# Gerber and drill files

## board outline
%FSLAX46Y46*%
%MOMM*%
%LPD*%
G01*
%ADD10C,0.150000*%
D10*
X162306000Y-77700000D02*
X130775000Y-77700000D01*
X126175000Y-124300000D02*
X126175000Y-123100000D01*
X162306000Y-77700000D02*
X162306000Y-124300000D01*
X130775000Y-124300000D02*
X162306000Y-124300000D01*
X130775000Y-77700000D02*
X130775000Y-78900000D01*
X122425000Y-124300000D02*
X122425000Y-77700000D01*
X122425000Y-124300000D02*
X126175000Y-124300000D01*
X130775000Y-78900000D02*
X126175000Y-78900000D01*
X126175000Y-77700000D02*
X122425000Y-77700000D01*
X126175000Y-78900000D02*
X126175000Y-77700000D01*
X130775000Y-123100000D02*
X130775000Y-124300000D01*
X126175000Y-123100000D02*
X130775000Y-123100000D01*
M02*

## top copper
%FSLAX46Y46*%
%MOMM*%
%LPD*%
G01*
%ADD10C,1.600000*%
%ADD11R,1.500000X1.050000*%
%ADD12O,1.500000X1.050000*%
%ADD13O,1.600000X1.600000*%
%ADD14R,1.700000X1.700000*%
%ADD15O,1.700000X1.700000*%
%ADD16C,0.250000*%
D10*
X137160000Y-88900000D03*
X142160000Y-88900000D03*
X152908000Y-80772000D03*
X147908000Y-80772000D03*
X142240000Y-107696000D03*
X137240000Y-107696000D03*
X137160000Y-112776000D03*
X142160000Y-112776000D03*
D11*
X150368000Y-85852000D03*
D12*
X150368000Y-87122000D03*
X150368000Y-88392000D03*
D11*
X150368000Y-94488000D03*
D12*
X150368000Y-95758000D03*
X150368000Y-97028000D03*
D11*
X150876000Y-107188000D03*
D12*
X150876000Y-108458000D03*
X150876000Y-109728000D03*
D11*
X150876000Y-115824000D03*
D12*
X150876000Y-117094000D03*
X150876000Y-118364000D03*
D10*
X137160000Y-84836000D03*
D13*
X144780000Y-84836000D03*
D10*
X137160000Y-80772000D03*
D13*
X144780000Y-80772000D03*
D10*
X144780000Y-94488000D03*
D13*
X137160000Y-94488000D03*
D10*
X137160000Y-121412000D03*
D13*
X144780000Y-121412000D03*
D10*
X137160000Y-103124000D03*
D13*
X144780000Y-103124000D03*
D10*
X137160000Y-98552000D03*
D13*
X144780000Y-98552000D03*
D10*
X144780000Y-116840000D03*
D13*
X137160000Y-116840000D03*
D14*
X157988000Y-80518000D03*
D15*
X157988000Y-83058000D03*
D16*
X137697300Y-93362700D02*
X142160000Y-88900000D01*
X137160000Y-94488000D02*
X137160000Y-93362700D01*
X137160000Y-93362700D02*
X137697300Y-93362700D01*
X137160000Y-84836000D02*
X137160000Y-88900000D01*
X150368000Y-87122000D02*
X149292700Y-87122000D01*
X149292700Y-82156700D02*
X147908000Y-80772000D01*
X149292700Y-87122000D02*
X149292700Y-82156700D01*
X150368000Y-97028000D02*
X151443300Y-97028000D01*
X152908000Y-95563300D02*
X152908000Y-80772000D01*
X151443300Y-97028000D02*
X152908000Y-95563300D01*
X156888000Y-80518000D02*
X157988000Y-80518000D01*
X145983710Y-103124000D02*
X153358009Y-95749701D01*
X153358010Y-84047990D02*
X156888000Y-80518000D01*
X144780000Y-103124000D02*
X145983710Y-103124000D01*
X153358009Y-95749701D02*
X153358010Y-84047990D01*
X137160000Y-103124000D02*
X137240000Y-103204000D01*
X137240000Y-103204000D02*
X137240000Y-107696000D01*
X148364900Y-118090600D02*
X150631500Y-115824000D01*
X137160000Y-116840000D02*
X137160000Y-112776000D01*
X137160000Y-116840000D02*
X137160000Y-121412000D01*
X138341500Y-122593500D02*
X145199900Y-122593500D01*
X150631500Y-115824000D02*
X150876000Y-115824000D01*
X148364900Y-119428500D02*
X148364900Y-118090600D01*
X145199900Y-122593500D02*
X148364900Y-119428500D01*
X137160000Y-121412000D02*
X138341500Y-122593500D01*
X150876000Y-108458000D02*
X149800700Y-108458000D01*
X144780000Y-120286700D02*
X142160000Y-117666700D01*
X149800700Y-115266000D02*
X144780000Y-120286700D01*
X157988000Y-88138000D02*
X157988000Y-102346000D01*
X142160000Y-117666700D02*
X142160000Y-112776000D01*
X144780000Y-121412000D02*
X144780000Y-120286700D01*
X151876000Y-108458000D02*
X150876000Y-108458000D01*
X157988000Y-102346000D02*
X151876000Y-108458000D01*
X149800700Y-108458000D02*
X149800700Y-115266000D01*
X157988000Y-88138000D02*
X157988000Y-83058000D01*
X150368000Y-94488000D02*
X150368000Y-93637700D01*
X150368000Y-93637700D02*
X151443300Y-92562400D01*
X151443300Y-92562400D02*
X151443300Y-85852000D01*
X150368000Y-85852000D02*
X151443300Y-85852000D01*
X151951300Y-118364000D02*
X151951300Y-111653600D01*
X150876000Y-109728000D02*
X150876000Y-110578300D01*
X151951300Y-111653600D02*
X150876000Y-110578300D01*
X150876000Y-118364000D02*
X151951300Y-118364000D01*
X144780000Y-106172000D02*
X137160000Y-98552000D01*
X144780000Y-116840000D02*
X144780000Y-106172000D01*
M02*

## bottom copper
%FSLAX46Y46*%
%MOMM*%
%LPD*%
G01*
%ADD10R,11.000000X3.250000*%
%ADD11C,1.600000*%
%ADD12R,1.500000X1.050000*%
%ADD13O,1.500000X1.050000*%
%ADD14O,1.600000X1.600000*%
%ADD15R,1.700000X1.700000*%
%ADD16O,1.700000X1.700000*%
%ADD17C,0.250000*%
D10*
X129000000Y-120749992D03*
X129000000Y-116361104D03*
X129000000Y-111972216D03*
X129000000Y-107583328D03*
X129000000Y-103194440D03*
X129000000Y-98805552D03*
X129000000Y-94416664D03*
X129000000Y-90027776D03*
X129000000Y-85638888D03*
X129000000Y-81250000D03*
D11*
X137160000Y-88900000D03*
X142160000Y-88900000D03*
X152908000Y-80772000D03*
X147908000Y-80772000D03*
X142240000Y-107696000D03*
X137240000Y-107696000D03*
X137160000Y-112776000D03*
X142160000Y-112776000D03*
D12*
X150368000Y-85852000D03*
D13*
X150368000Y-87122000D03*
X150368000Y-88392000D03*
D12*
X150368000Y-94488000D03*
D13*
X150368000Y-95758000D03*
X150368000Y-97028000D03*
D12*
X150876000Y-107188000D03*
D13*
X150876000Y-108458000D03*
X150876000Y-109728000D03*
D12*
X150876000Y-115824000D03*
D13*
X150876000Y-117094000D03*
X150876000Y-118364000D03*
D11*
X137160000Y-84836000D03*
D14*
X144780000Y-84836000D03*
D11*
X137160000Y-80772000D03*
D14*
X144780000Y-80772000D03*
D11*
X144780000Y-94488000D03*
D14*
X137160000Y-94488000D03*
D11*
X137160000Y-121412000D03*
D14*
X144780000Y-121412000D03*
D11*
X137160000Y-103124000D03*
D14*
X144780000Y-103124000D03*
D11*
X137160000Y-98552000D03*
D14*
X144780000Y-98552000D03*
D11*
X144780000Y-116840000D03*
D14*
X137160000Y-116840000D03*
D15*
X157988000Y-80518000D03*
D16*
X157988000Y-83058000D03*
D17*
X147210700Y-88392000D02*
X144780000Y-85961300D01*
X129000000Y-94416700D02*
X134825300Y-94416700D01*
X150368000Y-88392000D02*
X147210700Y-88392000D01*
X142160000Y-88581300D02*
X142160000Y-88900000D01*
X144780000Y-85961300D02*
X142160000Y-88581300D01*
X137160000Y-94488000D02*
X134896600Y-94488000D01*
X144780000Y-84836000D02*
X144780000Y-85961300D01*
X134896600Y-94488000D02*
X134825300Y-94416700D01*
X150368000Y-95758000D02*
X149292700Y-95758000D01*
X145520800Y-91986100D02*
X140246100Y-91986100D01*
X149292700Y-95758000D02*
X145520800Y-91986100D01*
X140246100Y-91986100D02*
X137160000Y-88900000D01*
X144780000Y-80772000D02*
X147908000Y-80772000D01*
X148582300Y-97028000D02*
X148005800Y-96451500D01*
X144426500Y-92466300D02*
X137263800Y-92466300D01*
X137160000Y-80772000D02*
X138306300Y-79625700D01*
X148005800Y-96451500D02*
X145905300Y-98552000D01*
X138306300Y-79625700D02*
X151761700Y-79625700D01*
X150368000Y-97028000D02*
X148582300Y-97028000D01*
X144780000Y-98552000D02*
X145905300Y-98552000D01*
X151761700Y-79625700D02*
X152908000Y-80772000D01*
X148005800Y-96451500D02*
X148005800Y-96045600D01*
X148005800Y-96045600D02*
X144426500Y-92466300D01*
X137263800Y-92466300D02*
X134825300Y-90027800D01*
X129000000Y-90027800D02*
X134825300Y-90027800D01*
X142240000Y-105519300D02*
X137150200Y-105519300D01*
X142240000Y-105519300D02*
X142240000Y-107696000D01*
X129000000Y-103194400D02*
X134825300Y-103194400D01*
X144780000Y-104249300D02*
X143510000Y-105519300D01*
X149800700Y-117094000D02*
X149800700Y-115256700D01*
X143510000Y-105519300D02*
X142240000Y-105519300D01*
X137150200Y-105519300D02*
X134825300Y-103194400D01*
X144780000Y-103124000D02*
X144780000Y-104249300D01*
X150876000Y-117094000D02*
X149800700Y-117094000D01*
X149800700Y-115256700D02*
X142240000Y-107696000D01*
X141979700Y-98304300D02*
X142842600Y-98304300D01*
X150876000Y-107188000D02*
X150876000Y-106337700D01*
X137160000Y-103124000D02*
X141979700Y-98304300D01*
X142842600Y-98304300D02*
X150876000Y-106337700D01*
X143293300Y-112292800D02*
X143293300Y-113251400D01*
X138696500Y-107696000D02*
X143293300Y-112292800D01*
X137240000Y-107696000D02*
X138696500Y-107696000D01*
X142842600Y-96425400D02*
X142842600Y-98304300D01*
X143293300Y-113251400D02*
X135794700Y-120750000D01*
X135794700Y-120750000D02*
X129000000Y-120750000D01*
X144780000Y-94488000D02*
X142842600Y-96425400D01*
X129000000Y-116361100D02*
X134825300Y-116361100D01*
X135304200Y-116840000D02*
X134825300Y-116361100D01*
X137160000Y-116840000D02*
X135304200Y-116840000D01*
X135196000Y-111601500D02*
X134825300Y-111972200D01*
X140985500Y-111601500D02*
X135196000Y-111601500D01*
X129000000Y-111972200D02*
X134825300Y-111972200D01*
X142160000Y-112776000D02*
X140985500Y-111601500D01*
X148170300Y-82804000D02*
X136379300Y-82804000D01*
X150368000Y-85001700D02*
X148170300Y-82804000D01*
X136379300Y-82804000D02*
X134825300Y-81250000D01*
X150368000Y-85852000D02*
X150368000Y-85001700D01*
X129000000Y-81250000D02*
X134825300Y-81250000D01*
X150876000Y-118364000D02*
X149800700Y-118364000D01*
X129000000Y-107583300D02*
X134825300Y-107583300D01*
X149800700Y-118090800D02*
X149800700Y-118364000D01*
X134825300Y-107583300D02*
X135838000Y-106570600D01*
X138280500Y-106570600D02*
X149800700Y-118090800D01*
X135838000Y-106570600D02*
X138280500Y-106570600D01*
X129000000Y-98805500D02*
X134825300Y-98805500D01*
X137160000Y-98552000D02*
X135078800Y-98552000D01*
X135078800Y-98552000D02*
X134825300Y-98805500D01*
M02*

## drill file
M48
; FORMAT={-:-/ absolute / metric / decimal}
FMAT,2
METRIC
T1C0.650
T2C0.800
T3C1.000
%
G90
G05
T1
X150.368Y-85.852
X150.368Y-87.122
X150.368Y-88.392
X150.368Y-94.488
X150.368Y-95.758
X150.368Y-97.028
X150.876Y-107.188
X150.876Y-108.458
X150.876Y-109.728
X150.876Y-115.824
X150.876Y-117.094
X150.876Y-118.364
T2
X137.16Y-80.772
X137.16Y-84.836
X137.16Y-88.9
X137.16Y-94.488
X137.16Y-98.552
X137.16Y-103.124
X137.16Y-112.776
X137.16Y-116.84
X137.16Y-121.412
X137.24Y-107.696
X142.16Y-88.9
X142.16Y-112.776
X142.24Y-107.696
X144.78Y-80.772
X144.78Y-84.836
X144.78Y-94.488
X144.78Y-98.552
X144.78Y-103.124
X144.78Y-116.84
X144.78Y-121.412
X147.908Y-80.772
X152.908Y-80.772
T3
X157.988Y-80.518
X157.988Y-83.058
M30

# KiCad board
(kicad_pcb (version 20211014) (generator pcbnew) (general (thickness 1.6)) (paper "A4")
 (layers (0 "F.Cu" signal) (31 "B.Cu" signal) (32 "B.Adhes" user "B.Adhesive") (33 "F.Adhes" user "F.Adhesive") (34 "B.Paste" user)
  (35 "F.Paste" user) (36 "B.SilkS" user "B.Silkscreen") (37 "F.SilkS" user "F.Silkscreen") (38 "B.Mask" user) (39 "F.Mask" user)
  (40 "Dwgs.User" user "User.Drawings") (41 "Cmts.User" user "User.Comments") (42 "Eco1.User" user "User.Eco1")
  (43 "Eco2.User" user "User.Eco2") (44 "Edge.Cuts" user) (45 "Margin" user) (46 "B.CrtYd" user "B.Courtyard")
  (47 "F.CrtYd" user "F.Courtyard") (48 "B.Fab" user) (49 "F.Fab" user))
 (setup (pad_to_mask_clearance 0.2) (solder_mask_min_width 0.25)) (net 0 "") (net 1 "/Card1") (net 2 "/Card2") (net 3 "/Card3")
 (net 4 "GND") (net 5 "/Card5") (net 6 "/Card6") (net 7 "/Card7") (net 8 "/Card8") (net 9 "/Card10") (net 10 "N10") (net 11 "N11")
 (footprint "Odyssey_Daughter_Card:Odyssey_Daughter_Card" (layer "F.Cu") (at 129 101)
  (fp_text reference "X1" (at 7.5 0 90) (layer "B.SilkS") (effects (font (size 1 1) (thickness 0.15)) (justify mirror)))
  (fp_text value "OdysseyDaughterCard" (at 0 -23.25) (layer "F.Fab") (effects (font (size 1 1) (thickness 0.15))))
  (pad "1" smd rect locked (at 0 19.749992) (size 11 3.25) (layers "B.Cu" "B.Mask") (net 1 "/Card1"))
  (pad "2" smd rect locked (at 0 15.361104) (size 11 3.25) (layers "B.Cu" "B.Mask") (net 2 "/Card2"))
  (pad "3" smd rect locked (at 0 10.972216) (size 11 3.25) (layers "B.Cu" "B.Mask") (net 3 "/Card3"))
  (pad "4" smd rect locked (at 0 6.583328) (size 11 3.25) (layers "B.Cu" "B.Mask") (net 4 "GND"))
  (pad "5" smd rect locked (at 0 2.19444) (size 11 3.25) (layers "B.Cu" "B.Mask") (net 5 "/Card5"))
  (pad "6" smd rect locked (at 0 -2.194448) (size 11 3.25) (layers "B.Cu" "B.Mask") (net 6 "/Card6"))
  (pad "7" smd rect locked (at 0 -6.583336) (size 11 3.25) (layers "B.Cu" "B.Mask") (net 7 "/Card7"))
  (pad "8" smd rect locked (at 0 -10.972224) (size 11 3.25) (layers "B.Cu" "B.Mask") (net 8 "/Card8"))
  (pad "9" smd rect locked (at 0 -15.361112) (size 11 3.25) (layers "B.Cu" "B.Mask"))
  (pad "10" smd rect locked (at 0 -19.75) (size 11 3.25) (layers "B.Cu" "B.Mask") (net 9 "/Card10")))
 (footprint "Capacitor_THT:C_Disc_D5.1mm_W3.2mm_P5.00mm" (layer "F.Cu") (at 137.16 88.9)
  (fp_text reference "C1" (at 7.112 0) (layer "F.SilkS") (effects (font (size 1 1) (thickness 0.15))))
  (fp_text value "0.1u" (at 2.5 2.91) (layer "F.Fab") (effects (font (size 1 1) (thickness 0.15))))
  (pad "1" thru_hole circle locked (at 0 0) (size 1.6 1.6) (drill 0.8) (layers *.Cu *.Mask) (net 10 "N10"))
  (pad "2" thru_hole circle locked (at 5 0) (size 1.6 1.6) (drill 0.8) (layers *.Cu *.Mask) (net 7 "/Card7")))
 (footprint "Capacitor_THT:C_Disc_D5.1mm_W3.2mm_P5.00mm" (layer "F.Cu") (at 152.908 80.772 180)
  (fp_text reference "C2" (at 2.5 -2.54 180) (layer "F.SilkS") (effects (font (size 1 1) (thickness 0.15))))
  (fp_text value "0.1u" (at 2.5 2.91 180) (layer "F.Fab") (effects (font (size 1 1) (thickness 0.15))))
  (pad "1" thru_hole circle locked (at 0 0 180) (size 1.6 1.6) (drill 0.8) (layers *.Cu *.Mask) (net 8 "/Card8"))
  (pad "2" thru_hole circle locked (at 5 0 180) (size 1.6 1.6) (drill 0.8) (layers *.Cu *.Mask) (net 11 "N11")))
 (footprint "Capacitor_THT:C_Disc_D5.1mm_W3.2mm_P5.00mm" (layer "F.Cu") (at 142.24 107.696 180)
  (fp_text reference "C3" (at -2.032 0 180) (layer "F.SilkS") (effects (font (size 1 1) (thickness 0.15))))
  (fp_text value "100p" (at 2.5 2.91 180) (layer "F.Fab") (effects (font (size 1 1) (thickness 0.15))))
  (pad "1" thru_hole circle locked (at 0 0 180) (size 1.6 1.6) (drill 0.8) (layers *.Cu *.Mask) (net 5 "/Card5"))
  (pad "2" thru_hole circle locked (at 5 0 180) (size 1.6 1.6) (drill 0.8) (layers *.Cu *.Mask) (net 1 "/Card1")))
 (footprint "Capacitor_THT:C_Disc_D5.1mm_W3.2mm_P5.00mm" (layer "F.Cu") (at 137.16 112.776)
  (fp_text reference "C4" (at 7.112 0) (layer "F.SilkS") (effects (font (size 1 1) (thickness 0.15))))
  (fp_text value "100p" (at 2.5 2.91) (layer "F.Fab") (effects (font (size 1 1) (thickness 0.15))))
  (pad "1" thru_hole circle locked (at 0 0) (size 1.6 1.6) (drill 0.8) (layers *.Cu *.Mask) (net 2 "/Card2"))
  (pad "2" thru_hole circle locked (at 5 0) (size 1.6 1.6) (drill 0.8) (layers *.Cu *.Mask) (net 3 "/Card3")))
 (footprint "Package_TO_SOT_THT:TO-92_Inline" (layer "F.Cu") (at 150.368 85.852 -90)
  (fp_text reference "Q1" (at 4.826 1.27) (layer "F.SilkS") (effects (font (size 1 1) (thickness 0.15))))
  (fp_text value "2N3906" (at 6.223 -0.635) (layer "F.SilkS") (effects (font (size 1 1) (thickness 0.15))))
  (pad "1" thru_hole rect locked (at 0 0 270) (size 1.05 1.5) (drill 0.65) (layers *.Cu *.Mask) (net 9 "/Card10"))
  (pad "2" thru_hole oval locked (at 1.27 0 270) (size 1.05 1.5) (drill 0.65) (layers *.Cu *.Mask) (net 11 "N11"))
  (pad "3" thru_hole oval locked (at 2.54 0 270) (size 1.05 1.5) (drill 0.65) (layers *.Cu *.Mask) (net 7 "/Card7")))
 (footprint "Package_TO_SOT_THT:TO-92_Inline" (layer "F.Cu") (at 150.368 94.488 -90)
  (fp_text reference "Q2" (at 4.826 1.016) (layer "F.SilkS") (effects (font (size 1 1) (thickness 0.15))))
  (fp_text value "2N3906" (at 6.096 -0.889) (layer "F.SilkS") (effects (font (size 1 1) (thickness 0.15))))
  (pad "1" thru_hole rect locked (at 0 0 270) (size 1.05 1.5) (drill 0.65) (layers *.Cu *.Mask) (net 9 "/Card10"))
  (pad "2" thru_hole oval locked (at 1.27 0 270) (size 1.05 1.5) (drill 0.65) (layers *.Cu *.Mask) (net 10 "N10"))
  (pad "3" thru_hole oval locked (at 2.54 0 270) (size 1.05 1.5) (drill 0.65) (layers *.Cu *.Mask) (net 8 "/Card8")))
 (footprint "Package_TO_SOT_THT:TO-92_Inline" (layer "F.Cu") (at 150.876 107.188 -90)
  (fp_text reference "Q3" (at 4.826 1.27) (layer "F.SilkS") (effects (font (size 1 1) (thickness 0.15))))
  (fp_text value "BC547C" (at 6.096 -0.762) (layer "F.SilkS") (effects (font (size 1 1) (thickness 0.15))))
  (pad "1" thru_hole rect locked (at 0 0 270) (size 1.05 1.5) (drill 0.65) (layers *.Cu *.Mask) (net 1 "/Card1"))
  (pad "2" thru_hole oval locked (at 1.27 0 270) (size 1.05 1.5) (drill 0.65) (layers *.Cu *.Mask) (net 3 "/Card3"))
  (pad "3" thru_hole oval locked (at 2.54 0 270) (size 1.05 1.5) (drill 0.65) (layers *.Cu *.Mask) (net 4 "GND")))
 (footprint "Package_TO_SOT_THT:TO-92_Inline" (layer "F.Cu") (at 150.876 115.824 -90)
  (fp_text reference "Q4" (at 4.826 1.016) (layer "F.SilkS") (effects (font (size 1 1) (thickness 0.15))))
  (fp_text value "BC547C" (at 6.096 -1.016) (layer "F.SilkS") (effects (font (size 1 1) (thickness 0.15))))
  (pad "1" thru_hole rect locked (at 0 0 270) (size 1.05 1.5) (drill 0.65) (layers *.Cu *.Mask) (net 2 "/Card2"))
  (pad "2" thru_hole oval locked (at 1.27 0 270) (size 1.05 1.5) (drill 0.65) (layers *.Cu *.Mask) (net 5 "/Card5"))
  (pad "3" thru_hole oval locked (at 2.54 0 270) (size 1.05 1.5) (drill 0.65) (layers *.Cu *.Mask) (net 4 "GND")))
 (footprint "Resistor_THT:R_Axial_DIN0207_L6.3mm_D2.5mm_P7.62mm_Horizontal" (layer "F.Cu") (at 137.16 84.836)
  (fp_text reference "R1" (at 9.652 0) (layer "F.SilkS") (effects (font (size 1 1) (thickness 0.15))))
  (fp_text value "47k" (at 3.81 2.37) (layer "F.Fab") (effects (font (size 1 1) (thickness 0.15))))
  (pad "1" thru_hole circle locked (at 0 0) (size 1.6 1.6) (drill 0.8) (layers *.Cu *.Mask) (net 10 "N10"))
  (pad "2" thru_hole oval locked (at 7.62 0) (size 1.6 1.6) (drill 0.8) (layers *.Cu *.Mask) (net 7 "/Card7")))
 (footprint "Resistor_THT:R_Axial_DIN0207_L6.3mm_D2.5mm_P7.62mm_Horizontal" (layer "F.Cu") (at 137.16 80.772)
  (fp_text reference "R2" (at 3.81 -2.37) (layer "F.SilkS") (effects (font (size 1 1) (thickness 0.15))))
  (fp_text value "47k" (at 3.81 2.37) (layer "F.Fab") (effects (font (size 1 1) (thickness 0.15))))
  (pad "1" thru_hole circle locked (at 0 0) (size 1.6 1.6) (drill 0.8) (layers *.Cu *.Mask) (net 8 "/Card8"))
  (pad "2" thru_hole oval locked (at 7.62 0) (size 1.6 1.6) (drill 0.8) (layers *.Cu *.Mask) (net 11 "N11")))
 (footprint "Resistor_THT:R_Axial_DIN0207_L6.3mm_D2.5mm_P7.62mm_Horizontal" (layer "F.Cu") (at 144.78 94.488 180)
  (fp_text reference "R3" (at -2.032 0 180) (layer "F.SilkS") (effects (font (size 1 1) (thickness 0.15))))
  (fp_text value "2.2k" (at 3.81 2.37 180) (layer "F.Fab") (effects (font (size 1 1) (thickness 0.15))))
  (pad "1" thru_hole circle locked (at 0 0 180) (size 1.6 1.6) (drill 0.8) (layers *.Cu *.Mask) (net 1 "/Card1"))
  (pad "2" thru_hole oval locked (at 7.62 0 180) (size 1.6 1.6) (drill 0.8) (layers *.Cu *.Mask) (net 7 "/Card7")))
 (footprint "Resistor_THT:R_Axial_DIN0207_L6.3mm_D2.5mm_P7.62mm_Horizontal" (layer "F.Cu") (at 137.16 121.412)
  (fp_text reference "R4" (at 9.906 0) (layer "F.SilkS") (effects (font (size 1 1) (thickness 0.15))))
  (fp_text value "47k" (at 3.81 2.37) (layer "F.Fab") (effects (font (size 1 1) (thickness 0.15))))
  (pad "1" thru_hole circle locked (at 0 0) (size 1.6 1.6) (drill 0.8) (layers *.Cu *.Mask) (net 2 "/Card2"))
  (pad "2" thru_hole oval locked (at 7.62 0) (size 1.6 1.6) (drill 0.8) (layers *.Cu *.Mask) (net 3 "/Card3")))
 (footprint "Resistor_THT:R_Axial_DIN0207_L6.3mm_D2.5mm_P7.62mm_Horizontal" (layer "F.Cu") (at 137.16 103.124)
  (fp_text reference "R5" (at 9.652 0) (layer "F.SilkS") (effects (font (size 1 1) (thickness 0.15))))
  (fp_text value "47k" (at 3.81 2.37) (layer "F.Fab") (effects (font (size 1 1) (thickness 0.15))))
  (pad "1" thru_hole circle locked (at 0 0) (size 1.6 1.6) (drill 0.8) (layers *.Cu *.Mask) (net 1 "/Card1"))
  (pad "2" thru_hole oval locked (at 7.62 0) (size 1.6 1.6) (drill 0.8) (layers *.Cu *.Mask) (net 5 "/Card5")))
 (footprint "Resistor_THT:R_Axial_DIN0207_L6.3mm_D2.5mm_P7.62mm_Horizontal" (layer "F.Cu") (at 137.16 98.552)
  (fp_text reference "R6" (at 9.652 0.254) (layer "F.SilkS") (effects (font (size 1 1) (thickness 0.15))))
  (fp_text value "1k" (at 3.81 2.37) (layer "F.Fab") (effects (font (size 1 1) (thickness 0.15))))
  (pad "1" thru_hole circle locked (at 0 0) (size 1.6 1.6) (drill 0.8) (layers *.Cu *.Mask) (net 6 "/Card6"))
  (pad "2" thru_hole oval locked (at 7.62 0) (size 1.6 1.6) (drill 0.8) (layers *.Cu *.Mask) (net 8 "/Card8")))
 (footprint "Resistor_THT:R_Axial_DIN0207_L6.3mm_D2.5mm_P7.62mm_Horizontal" (layer "F.Cu") (at 144.78 116.84 180)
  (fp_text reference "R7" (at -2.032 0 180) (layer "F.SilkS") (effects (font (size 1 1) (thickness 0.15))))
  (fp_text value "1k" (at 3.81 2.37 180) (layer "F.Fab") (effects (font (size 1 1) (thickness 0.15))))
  (pad "1" thru_hole circle locked (at 0 0 180) (size 1.6 1.6) (drill 0.8) (layers *.Cu *.Mask) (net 6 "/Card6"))
  (pad "2" thru_hole oval locked (at 7.62 0 180) (size 1.6 1.6) (drill 0.8) (layers *.Cu *.Mask) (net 2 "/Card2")))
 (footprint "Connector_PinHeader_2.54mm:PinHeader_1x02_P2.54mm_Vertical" (layer "F.Cu") (at 157.988 80.518)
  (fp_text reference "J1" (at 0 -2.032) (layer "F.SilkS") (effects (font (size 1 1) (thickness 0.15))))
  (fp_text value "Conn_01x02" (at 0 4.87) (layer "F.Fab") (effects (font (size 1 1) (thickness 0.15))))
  (pad "1" thru_hole rect locked (at 0 0) (size 1.7 1.7) (drill 1) (layers *.Cu *.Mask) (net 5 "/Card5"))
  (pad "2" thru_hole oval locked (at 0 2.54) (size 1.7 1.7) (drill 1) (layers *.Cu *.Mask) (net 3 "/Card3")))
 (gr_line (start 162.306 77.7) (end 130.775 77.7) (layer "Edge.Cuts") (width 0.15))
 (gr_line (start 126.175 124.3) (end 126.175 123.1) (layer "Edge.Cuts") (width 0.15))
 (gr_line (start 162.306 77.7) (end 162.306 124.3) (layer "Edge.Cuts") (width 0.15))
 (gr_line (start 130.775 124.3) (end 162.306 124.3) (layer "Edge.Cuts") (width 0.15))
 (gr_line (start 130.775 77.7) (end 130.775 78.9) (layer "Edge.Cuts") (width 0.15))
 (gr_line (start 122.425 124.3) (end 122.425 77.7) (layer "Edge.Cuts") (width 0.15))
 (gr_line (start 122.425 124.3) (end 126.175 124.3) (layer "Edge.Cuts") (width 0.15))
 (gr_line (start 130.775 78.9) (end 126.175 78.9) (layer "Edge.Cuts") (width 0.15))
 (gr_line (start 126.175 77.7) (end 122.425 77.7) (layer "Edge.Cuts") (width 0.15))
 (gr_line (start 126.175 78.9) (end 126.175 77.7) (layer "Edge.Cuts") (width 0.15))
 (gr_line (start 130.775 123.1) (end 130.775 124.3) (layer "Edge.Cuts") (width 0.15))
 (gr_line (start 126.175 123.1) (end 130.775 123.1) (layer "Edge.Cuts") (width 0.15))
 (segment (start 137.6973 93.3627) (end 142.16 88.9) (width 0.25) (layer "F.Cu") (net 7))
 (segment (start 137.16 94.488) (end 137.16 93.3627) (width 0.25) (layer "F.Cu") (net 7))
 (segment (start 137.16 93.3627) (end 137.6973 93.3627) (width 0.25) (layer "F.Cu") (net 7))
 (segment (start 147.2107 88.392) (end 144.78 85.9613) (width 0.25) (layer "B.Cu") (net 7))
 (segment (start 129 94.4167) (end 134.8253 94.4167) (width 0.25) (layer "B.Cu") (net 7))
 (segment (start 150.368 88.392) (end 147.2107 88.392) (width 0.25) (layer "B.Cu") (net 7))
 (segment (start 142.16 88.5813) (end 142.16 88.9) (width 0.25) (layer "B.Cu") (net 7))
 (segment (start 144.78 85.9613) (end 142.16 88.5813) (width 0.25) (layer "B.Cu") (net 7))
 (segment (start 137.16 94.488) (end 134.8966 94.488) (width 0.25) (layer "B.Cu") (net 7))
 (segment (start 144.78 84.836) (end 144.78 85.9613) (width 0.25) (layer "B.Cu") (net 7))
 (segment (start 134.8966 94.488) (end 134.8253 94.4167) (width 0.25) (layer "B.Cu") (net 7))
 (segment (start 137.16 84.836) (end 137.16 88.9) (width 0.25) (layer "F.Cu") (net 10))
 (segment (start 150.368 95.758) (end 149.2927 95.758) (width 0.25) (layer "B.Cu") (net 10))
 (segment (start 145.5208 91.9861) (end 140.2461 91.9861) (width 0.25) (layer "B.Cu") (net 10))
 (segment (start 149.2927 95.758) (end 145.5208 91.9861) (width 0.25) (layer "B.Cu") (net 10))
 (segment (start 140.2461 91.9861) (end 137.16 88.9) (width 0.25) (layer "B.Cu") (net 10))
 (segment (start 150.368 87.122) (end 149.2927 87.122) (width 0.25) (layer "F.Cu") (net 11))
 (segment (start 149.2927 82.1567) (end 147.908 80.772) (width 0.25) (layer "F.Cu") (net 11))
 (segment (start 149.2927 87.122) (end 149.2927 82.1567) (width 0.25) (layer "F.Cu") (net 11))
 (segment (start 144.78 80.772) (end 147.908 80.772) (width 0.25) (layer "B.Cu") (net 11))
 (segment (start 150.368 97.028) (end 151.4433 97.028) (width 0.25) (layer "F.Cu") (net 8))
 (segment (start 152.908 95.5633) (end 152.908 80.772) (width 0.25) (layer "F.Cu") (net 8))
 (segment (start 151.4433 97.028) (end 152.908 95.5633) (width 0.25) (layer "F.Cu") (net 8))
 (segment (start 148.5823 97.028) (end 148.0058 96.4515) (width 0.25) (layer "B.Cu") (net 8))
 (segment (start 144.4265 92.4663) (end 137.2638 92.4663) (width 0.25) (layer "B.Cu") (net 8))
 (segment (start 137.16 80.772) (end 138.3063 79.6257) (width 0.25) (layer "B.Cu") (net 8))
 (segment (start 148.0058 96.4515) (end 145.9053 98.552) (width 0.25) (layer "B.Cu") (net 8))
 (segment (start 138.3063 79.6257) (end 151.7617 79.6257) (width 0.25) (layer "B.Cu") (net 8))
 (segment (start 150.368 97.028) (end 148.5823 97.028) (width 0.25) (layer "B.Cu") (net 8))
 (segment (start 144.78 98.552) (end 145.9053 98.552) (width 0.25) (layer "B.Cu") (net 8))
 (segment (start 151.7617 79.6257) (end 152.908 80.772) (width 0.25) (layer "B.Cu") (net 8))
 (segment (start 148.0058 96.4515) (end 148.0058 96.0456) (width 0.25) (layer "B.Cu") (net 8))
 (segment (start 148.0058 96.0456) (end 144.4265 92.4663) (width 0.25) (layer "B.Cu") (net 8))
 (segment (start 137.2638 92.4663) (end 134.8253 90.0278) (width 0.25) (layer "B.Cu") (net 8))
 (segment (start 129 90.0278) (end 134.8253 90.0278) (width 0.25) (layer "B.Cu") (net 8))
 (segment (start 156.888 80.518) (end 157.988 80.518) (width 0.25) (layer "F.Cu") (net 5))
 (segment (start 145.98371 103.124) (end 153.358009 95.749701) (width 0.25) (layer "F.Cu") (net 5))
 (segment (start 153.35801 84.04799) (end 156.888 80.518) (width 0.25) (layer "F.Cu") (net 5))
 (segment (start 144.78 103.124) (end 145.98371 103.124) (width 0.25) (layer "F.Cu") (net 5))
 (segment (start 153.358009 95.749701) (end 153.35801 84.04799) (width 0.25) (layer "F.Cu") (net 5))
 (segment (start 142.24 105.5193) (end 137.1502 105.5193) (width 0.25) (layer "B.Cu") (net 5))
 (segment (start 142.24 105.5193) (end 142.24 107.696) (width 0.25) (layer "B.Cu") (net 5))
 (segment (start 129 103.1944) (end 134.8253 103.1944) (width 0.25) (layer "B.Cu") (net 5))
 (segment (start 144.78 104.2493) (end 143.51 105.5193) (width 0.25) (layer "B.Cu") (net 5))
 (segment (start 149.8007 117.094) (end 149.8007 115.2567) (width 0.25) (layer "B.Cu") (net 5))
 (segment (start 143.51 105.5193) (end 142.24 105.5193) (width 0.25) (layer "B.Cu") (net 5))
 (segment (start 137.1502 105.5193) (end 134.8253 103.1944) (width 0.25) (layer "B.Cu") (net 5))
 (segment (start 144.78 103.124) (end 144.78 104.2493) (width 0.25) (layer "B.Cu") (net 5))
 (segment (start 150.876 117.094) (end 149.8007 117.094) (width 0.25) (layer "B.Cu") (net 5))
 (segment (start 149.8007 115.2567) (end 142.24 107.696) (width 0.25) (layer "B.Cu") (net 5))
 (segment (start 137.16 103.124) (end 137.24 103.204) (width 0.25) (layer "F.Cu") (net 1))
 (segment (start 137.24 103.204) (end 137.24 107.696) (width 0.25) (layer "F.Cu") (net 1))
 (segment (start 141.9797 98.3043) (end 142.8426 98.3043) (width 0.25) (layer "B.Cu") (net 1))
 (segment (start 150.876 107.188) (end 150.876 106.3377) (width 0.25) (layer "B.Cu") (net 1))
 (segment (start 137.16 103.124) (end 141.9797 98.3043) (width 0.25) (layer "B.Cu") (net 1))
 (segment (start 142.8426 98.3043) (end 150.876 106.3377) (width 0.25) (layer "B.Cu") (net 1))
 (segment (start 143.2933 112.2928) (end 143.2933 113.2514) (width 0.25) (layer "B.Cu") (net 1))
 (segment (start 138.6965 107.696) (end 143.2933 112.2928) (width 0.25) (layer "B.Cu") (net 1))
 (segment (start 137.24 107.696) (end 138.6965 107.696) (width 0.25) (layer "B.Cu") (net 1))
 (segment (start 142.8426 96.4254) (end 142.8426 98.3043) (width 0.25) (layer "B.Cu") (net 1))
 (segment (start 143.2933 113.2514) (end 135.7947 120.75) (width 0.25) (layer "B.Cu") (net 1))
 (segment (start 135.7947 120.75) (end 129 120.75) (width 0.25) (layer "B.Cu") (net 1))
 (segment (start 144.78 94.488) (end 142.8426 96.4254) (width 0.25) (layer "B.Cu") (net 1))
 (segment (start 148.3649 118.0906) (end 150.6315 115.824) (width 0.25) (layer "F.Cu") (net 2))
 (segment (start 137.16 116.84) (end 137.16 112.776) (width 0.25) (layer "F.Cu") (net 2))
 (segment (start 137.16 116.84) (end 137.16 121.412) (width 0.25) (layer "F.Cu") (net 2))
 (segment (start 138.3415 122.5935) (end 145.1999 122.5935) (width 0.25) (layer "F.Cu") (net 2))
 (segment (start 150.6315 115.824) (end 150.876 115.824) (width 0.25) (layer "F.Cu") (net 2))
 (segment (start 148.3649 119.4285) (end 148.3649 118.0906) (width 0.25) (layer "F.Cu") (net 2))
 (segment (start 145.1999 122.5935) (end 148.3649 119.4285) (width 0.25) (layer "F.Cu") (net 2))
 (segment (start 137.16 121.412) (end 138.3415 122.5935) (width 0.25) (layer "F.Cu") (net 2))
 (segment (start 129 116.3611) (end 134.8253 116.3611) (width 0.25) (layer "B.Cu") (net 2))
 (segment (start 135.3042 116.84) (end 134.8253 116.3611) (width 0.25) (layer "B.Cu") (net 2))
 (segment (start 137.16 116.84) (end 135.3042 116.84) (width 0.25) (layer "B.Cu") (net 2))
 (segment (start 150.876 108.458) (end 149.8007 108.458) (width 0.25) (layer "F.Cu") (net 3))
 (segment (start 144.78 120.2867) (end 142.16 117.6667) (width 0.25) (layer "F.Cu") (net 3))
 (segment (start 149.8007 115.266) (end 144.78 120.2867) (width 0.25) (layer "F.Cu") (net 3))
 (segment (start 157.988 88.138) (end 157.988 102.346) (width 0.25) (layer "F.Cu") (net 3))
 (segment (start 142.16 117.6667) (end 142.16 112.776) (width 0.25) (layer "F.Cu") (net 3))
 (segment (start 144.78 121.412) (end 144.78 120.2867) (width 0.25) (layer "F.Cu") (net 3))
 (segment (start 151.876 108.458) (end 150.876 108.458) (width 0.25) (layer "F.Cu") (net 3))
 (segment (start 157.988 102.346) (end 151.876 108.458) (width 0.25) (layer "F.Cu") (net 3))
 (segment (start 149.8007 108.458) (end 149.8007 115.266) (width 0.25) (layer "F.Cu") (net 3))
 (segment (start 157.988 88.138) (end 157.988 83.058) (width 0.25) (layer "F.Cu") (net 3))
 (segment (start 135.196 111.6015) (end 134.8253 111.9722) (width 0.25) (layer "B.Cu") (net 3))
 (segment (start 140.9855 111.6015) (end 135.196 111.6015) (width 0.25) (layer "B.Cu") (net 3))
 (segment (start 129 111.9722) (end 134.8253 111.9722) (width 0.25) (layer "B.Cu") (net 3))
 (segment (start 142.16 112.776) (end 140.9855 111.6015) (width 0.25) (layer "B.Cu") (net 3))
 (segment (start 150.368 94.488) (end 150.368 93.6377) (width 0.25) (layer "F.Cu") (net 9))
 (segment (start 150.368 93.6377) (end 151.4433 92.5624) (width 0.25) (layer "F.Cu") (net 9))
 (segment (start 151.4433 92.5624) (end 151.4433 85.852) (width 0.25) (layer "F.Cu") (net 9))
 (segment (start 150.368 85.852) (end 151.4433 85.852) (width 0.25) (layer "F.Cu") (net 9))
 (segment (start 148.1703 82.804) (end 136.3793 82.804) (width 0.25) (layer "B.Cu") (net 9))
 (segment (start 150.368 85.0017) (end 148.1703 82.804) (width 0.25) (layer "B.Cu") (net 9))
 (segment (start 136.3793 82.804) (end 134.8253 81.25) (width 0.25) (layer "B.Cu") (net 9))
 (segment (start 150.368 85.852) (end 150.368 85.0017) (width 0.25) (layer "B.Cu") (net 9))
 (segment (start 129 81.25) (end 134.8253 81.25) (width 0.25) (layer "B.Cu") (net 9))
 (segment (start 151.9513 118.364) (end 151.9513 111.6536) (width 0.25) (layer "F.Cu") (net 4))
 (segment (start 150.876 109.728) (end 150.876 110.5783) (width 0.25) (layer "F.Cu") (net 4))
 (segment (start 151.9513 111.6536) (end 150.876 110.5783) (width 0.25) (layer "F.Cu") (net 4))
 (segment (start 150.876 118.364) (end 151.9513 118.364) (width 0.25) (layer "F.Cu") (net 4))
 (segment (start 150.876 118.364) (end 149.8007 118.364) (width 0.25) (layer "B.Cu") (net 4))
 (segment (start 129 107.5833) (end 134.8253 107.5833) (width 0.25) (layer "B.Cu") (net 4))
 (segment (start 149.8007 118.0908) (end 149.8007 118.364) (width 0.25) (layer "B.Cu") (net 4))
 (segment (start 134.8253 107.5833) (end 135.838 106.5706) (width 0.25) (layer "B.Cu") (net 4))
 (segment (start 138.2805 106.5706) (end 149.8007 118.0908) (width 0.25) (layer "B.Cu") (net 4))
 (segment (start 135.838 106.5706) (end 138.2805 106.5706) (width 0.25) (layer "B.Cu") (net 4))
 (segment (start 144.78 106.172) (end 137.16 98.552) (width 0.25) (layer "F.Cu") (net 6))
 (segment (start 144.78 116.84) (end 144.78 106.172) (width 0.25) (layer "F.Cu") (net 6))
 (segment (start 129 98.8055) (end 134.8253 98.8055) (width 0.25) (layer "B.Cu") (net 6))
 (segment (start 137.16 98.552) (end 135.0788 98.552) (width 0.25) (layer "B.Cu") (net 6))
 (segment (start 135.0788 98.552) (end 134.8253 98.8055) (width 0.25) (layer "B.Cu") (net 6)))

